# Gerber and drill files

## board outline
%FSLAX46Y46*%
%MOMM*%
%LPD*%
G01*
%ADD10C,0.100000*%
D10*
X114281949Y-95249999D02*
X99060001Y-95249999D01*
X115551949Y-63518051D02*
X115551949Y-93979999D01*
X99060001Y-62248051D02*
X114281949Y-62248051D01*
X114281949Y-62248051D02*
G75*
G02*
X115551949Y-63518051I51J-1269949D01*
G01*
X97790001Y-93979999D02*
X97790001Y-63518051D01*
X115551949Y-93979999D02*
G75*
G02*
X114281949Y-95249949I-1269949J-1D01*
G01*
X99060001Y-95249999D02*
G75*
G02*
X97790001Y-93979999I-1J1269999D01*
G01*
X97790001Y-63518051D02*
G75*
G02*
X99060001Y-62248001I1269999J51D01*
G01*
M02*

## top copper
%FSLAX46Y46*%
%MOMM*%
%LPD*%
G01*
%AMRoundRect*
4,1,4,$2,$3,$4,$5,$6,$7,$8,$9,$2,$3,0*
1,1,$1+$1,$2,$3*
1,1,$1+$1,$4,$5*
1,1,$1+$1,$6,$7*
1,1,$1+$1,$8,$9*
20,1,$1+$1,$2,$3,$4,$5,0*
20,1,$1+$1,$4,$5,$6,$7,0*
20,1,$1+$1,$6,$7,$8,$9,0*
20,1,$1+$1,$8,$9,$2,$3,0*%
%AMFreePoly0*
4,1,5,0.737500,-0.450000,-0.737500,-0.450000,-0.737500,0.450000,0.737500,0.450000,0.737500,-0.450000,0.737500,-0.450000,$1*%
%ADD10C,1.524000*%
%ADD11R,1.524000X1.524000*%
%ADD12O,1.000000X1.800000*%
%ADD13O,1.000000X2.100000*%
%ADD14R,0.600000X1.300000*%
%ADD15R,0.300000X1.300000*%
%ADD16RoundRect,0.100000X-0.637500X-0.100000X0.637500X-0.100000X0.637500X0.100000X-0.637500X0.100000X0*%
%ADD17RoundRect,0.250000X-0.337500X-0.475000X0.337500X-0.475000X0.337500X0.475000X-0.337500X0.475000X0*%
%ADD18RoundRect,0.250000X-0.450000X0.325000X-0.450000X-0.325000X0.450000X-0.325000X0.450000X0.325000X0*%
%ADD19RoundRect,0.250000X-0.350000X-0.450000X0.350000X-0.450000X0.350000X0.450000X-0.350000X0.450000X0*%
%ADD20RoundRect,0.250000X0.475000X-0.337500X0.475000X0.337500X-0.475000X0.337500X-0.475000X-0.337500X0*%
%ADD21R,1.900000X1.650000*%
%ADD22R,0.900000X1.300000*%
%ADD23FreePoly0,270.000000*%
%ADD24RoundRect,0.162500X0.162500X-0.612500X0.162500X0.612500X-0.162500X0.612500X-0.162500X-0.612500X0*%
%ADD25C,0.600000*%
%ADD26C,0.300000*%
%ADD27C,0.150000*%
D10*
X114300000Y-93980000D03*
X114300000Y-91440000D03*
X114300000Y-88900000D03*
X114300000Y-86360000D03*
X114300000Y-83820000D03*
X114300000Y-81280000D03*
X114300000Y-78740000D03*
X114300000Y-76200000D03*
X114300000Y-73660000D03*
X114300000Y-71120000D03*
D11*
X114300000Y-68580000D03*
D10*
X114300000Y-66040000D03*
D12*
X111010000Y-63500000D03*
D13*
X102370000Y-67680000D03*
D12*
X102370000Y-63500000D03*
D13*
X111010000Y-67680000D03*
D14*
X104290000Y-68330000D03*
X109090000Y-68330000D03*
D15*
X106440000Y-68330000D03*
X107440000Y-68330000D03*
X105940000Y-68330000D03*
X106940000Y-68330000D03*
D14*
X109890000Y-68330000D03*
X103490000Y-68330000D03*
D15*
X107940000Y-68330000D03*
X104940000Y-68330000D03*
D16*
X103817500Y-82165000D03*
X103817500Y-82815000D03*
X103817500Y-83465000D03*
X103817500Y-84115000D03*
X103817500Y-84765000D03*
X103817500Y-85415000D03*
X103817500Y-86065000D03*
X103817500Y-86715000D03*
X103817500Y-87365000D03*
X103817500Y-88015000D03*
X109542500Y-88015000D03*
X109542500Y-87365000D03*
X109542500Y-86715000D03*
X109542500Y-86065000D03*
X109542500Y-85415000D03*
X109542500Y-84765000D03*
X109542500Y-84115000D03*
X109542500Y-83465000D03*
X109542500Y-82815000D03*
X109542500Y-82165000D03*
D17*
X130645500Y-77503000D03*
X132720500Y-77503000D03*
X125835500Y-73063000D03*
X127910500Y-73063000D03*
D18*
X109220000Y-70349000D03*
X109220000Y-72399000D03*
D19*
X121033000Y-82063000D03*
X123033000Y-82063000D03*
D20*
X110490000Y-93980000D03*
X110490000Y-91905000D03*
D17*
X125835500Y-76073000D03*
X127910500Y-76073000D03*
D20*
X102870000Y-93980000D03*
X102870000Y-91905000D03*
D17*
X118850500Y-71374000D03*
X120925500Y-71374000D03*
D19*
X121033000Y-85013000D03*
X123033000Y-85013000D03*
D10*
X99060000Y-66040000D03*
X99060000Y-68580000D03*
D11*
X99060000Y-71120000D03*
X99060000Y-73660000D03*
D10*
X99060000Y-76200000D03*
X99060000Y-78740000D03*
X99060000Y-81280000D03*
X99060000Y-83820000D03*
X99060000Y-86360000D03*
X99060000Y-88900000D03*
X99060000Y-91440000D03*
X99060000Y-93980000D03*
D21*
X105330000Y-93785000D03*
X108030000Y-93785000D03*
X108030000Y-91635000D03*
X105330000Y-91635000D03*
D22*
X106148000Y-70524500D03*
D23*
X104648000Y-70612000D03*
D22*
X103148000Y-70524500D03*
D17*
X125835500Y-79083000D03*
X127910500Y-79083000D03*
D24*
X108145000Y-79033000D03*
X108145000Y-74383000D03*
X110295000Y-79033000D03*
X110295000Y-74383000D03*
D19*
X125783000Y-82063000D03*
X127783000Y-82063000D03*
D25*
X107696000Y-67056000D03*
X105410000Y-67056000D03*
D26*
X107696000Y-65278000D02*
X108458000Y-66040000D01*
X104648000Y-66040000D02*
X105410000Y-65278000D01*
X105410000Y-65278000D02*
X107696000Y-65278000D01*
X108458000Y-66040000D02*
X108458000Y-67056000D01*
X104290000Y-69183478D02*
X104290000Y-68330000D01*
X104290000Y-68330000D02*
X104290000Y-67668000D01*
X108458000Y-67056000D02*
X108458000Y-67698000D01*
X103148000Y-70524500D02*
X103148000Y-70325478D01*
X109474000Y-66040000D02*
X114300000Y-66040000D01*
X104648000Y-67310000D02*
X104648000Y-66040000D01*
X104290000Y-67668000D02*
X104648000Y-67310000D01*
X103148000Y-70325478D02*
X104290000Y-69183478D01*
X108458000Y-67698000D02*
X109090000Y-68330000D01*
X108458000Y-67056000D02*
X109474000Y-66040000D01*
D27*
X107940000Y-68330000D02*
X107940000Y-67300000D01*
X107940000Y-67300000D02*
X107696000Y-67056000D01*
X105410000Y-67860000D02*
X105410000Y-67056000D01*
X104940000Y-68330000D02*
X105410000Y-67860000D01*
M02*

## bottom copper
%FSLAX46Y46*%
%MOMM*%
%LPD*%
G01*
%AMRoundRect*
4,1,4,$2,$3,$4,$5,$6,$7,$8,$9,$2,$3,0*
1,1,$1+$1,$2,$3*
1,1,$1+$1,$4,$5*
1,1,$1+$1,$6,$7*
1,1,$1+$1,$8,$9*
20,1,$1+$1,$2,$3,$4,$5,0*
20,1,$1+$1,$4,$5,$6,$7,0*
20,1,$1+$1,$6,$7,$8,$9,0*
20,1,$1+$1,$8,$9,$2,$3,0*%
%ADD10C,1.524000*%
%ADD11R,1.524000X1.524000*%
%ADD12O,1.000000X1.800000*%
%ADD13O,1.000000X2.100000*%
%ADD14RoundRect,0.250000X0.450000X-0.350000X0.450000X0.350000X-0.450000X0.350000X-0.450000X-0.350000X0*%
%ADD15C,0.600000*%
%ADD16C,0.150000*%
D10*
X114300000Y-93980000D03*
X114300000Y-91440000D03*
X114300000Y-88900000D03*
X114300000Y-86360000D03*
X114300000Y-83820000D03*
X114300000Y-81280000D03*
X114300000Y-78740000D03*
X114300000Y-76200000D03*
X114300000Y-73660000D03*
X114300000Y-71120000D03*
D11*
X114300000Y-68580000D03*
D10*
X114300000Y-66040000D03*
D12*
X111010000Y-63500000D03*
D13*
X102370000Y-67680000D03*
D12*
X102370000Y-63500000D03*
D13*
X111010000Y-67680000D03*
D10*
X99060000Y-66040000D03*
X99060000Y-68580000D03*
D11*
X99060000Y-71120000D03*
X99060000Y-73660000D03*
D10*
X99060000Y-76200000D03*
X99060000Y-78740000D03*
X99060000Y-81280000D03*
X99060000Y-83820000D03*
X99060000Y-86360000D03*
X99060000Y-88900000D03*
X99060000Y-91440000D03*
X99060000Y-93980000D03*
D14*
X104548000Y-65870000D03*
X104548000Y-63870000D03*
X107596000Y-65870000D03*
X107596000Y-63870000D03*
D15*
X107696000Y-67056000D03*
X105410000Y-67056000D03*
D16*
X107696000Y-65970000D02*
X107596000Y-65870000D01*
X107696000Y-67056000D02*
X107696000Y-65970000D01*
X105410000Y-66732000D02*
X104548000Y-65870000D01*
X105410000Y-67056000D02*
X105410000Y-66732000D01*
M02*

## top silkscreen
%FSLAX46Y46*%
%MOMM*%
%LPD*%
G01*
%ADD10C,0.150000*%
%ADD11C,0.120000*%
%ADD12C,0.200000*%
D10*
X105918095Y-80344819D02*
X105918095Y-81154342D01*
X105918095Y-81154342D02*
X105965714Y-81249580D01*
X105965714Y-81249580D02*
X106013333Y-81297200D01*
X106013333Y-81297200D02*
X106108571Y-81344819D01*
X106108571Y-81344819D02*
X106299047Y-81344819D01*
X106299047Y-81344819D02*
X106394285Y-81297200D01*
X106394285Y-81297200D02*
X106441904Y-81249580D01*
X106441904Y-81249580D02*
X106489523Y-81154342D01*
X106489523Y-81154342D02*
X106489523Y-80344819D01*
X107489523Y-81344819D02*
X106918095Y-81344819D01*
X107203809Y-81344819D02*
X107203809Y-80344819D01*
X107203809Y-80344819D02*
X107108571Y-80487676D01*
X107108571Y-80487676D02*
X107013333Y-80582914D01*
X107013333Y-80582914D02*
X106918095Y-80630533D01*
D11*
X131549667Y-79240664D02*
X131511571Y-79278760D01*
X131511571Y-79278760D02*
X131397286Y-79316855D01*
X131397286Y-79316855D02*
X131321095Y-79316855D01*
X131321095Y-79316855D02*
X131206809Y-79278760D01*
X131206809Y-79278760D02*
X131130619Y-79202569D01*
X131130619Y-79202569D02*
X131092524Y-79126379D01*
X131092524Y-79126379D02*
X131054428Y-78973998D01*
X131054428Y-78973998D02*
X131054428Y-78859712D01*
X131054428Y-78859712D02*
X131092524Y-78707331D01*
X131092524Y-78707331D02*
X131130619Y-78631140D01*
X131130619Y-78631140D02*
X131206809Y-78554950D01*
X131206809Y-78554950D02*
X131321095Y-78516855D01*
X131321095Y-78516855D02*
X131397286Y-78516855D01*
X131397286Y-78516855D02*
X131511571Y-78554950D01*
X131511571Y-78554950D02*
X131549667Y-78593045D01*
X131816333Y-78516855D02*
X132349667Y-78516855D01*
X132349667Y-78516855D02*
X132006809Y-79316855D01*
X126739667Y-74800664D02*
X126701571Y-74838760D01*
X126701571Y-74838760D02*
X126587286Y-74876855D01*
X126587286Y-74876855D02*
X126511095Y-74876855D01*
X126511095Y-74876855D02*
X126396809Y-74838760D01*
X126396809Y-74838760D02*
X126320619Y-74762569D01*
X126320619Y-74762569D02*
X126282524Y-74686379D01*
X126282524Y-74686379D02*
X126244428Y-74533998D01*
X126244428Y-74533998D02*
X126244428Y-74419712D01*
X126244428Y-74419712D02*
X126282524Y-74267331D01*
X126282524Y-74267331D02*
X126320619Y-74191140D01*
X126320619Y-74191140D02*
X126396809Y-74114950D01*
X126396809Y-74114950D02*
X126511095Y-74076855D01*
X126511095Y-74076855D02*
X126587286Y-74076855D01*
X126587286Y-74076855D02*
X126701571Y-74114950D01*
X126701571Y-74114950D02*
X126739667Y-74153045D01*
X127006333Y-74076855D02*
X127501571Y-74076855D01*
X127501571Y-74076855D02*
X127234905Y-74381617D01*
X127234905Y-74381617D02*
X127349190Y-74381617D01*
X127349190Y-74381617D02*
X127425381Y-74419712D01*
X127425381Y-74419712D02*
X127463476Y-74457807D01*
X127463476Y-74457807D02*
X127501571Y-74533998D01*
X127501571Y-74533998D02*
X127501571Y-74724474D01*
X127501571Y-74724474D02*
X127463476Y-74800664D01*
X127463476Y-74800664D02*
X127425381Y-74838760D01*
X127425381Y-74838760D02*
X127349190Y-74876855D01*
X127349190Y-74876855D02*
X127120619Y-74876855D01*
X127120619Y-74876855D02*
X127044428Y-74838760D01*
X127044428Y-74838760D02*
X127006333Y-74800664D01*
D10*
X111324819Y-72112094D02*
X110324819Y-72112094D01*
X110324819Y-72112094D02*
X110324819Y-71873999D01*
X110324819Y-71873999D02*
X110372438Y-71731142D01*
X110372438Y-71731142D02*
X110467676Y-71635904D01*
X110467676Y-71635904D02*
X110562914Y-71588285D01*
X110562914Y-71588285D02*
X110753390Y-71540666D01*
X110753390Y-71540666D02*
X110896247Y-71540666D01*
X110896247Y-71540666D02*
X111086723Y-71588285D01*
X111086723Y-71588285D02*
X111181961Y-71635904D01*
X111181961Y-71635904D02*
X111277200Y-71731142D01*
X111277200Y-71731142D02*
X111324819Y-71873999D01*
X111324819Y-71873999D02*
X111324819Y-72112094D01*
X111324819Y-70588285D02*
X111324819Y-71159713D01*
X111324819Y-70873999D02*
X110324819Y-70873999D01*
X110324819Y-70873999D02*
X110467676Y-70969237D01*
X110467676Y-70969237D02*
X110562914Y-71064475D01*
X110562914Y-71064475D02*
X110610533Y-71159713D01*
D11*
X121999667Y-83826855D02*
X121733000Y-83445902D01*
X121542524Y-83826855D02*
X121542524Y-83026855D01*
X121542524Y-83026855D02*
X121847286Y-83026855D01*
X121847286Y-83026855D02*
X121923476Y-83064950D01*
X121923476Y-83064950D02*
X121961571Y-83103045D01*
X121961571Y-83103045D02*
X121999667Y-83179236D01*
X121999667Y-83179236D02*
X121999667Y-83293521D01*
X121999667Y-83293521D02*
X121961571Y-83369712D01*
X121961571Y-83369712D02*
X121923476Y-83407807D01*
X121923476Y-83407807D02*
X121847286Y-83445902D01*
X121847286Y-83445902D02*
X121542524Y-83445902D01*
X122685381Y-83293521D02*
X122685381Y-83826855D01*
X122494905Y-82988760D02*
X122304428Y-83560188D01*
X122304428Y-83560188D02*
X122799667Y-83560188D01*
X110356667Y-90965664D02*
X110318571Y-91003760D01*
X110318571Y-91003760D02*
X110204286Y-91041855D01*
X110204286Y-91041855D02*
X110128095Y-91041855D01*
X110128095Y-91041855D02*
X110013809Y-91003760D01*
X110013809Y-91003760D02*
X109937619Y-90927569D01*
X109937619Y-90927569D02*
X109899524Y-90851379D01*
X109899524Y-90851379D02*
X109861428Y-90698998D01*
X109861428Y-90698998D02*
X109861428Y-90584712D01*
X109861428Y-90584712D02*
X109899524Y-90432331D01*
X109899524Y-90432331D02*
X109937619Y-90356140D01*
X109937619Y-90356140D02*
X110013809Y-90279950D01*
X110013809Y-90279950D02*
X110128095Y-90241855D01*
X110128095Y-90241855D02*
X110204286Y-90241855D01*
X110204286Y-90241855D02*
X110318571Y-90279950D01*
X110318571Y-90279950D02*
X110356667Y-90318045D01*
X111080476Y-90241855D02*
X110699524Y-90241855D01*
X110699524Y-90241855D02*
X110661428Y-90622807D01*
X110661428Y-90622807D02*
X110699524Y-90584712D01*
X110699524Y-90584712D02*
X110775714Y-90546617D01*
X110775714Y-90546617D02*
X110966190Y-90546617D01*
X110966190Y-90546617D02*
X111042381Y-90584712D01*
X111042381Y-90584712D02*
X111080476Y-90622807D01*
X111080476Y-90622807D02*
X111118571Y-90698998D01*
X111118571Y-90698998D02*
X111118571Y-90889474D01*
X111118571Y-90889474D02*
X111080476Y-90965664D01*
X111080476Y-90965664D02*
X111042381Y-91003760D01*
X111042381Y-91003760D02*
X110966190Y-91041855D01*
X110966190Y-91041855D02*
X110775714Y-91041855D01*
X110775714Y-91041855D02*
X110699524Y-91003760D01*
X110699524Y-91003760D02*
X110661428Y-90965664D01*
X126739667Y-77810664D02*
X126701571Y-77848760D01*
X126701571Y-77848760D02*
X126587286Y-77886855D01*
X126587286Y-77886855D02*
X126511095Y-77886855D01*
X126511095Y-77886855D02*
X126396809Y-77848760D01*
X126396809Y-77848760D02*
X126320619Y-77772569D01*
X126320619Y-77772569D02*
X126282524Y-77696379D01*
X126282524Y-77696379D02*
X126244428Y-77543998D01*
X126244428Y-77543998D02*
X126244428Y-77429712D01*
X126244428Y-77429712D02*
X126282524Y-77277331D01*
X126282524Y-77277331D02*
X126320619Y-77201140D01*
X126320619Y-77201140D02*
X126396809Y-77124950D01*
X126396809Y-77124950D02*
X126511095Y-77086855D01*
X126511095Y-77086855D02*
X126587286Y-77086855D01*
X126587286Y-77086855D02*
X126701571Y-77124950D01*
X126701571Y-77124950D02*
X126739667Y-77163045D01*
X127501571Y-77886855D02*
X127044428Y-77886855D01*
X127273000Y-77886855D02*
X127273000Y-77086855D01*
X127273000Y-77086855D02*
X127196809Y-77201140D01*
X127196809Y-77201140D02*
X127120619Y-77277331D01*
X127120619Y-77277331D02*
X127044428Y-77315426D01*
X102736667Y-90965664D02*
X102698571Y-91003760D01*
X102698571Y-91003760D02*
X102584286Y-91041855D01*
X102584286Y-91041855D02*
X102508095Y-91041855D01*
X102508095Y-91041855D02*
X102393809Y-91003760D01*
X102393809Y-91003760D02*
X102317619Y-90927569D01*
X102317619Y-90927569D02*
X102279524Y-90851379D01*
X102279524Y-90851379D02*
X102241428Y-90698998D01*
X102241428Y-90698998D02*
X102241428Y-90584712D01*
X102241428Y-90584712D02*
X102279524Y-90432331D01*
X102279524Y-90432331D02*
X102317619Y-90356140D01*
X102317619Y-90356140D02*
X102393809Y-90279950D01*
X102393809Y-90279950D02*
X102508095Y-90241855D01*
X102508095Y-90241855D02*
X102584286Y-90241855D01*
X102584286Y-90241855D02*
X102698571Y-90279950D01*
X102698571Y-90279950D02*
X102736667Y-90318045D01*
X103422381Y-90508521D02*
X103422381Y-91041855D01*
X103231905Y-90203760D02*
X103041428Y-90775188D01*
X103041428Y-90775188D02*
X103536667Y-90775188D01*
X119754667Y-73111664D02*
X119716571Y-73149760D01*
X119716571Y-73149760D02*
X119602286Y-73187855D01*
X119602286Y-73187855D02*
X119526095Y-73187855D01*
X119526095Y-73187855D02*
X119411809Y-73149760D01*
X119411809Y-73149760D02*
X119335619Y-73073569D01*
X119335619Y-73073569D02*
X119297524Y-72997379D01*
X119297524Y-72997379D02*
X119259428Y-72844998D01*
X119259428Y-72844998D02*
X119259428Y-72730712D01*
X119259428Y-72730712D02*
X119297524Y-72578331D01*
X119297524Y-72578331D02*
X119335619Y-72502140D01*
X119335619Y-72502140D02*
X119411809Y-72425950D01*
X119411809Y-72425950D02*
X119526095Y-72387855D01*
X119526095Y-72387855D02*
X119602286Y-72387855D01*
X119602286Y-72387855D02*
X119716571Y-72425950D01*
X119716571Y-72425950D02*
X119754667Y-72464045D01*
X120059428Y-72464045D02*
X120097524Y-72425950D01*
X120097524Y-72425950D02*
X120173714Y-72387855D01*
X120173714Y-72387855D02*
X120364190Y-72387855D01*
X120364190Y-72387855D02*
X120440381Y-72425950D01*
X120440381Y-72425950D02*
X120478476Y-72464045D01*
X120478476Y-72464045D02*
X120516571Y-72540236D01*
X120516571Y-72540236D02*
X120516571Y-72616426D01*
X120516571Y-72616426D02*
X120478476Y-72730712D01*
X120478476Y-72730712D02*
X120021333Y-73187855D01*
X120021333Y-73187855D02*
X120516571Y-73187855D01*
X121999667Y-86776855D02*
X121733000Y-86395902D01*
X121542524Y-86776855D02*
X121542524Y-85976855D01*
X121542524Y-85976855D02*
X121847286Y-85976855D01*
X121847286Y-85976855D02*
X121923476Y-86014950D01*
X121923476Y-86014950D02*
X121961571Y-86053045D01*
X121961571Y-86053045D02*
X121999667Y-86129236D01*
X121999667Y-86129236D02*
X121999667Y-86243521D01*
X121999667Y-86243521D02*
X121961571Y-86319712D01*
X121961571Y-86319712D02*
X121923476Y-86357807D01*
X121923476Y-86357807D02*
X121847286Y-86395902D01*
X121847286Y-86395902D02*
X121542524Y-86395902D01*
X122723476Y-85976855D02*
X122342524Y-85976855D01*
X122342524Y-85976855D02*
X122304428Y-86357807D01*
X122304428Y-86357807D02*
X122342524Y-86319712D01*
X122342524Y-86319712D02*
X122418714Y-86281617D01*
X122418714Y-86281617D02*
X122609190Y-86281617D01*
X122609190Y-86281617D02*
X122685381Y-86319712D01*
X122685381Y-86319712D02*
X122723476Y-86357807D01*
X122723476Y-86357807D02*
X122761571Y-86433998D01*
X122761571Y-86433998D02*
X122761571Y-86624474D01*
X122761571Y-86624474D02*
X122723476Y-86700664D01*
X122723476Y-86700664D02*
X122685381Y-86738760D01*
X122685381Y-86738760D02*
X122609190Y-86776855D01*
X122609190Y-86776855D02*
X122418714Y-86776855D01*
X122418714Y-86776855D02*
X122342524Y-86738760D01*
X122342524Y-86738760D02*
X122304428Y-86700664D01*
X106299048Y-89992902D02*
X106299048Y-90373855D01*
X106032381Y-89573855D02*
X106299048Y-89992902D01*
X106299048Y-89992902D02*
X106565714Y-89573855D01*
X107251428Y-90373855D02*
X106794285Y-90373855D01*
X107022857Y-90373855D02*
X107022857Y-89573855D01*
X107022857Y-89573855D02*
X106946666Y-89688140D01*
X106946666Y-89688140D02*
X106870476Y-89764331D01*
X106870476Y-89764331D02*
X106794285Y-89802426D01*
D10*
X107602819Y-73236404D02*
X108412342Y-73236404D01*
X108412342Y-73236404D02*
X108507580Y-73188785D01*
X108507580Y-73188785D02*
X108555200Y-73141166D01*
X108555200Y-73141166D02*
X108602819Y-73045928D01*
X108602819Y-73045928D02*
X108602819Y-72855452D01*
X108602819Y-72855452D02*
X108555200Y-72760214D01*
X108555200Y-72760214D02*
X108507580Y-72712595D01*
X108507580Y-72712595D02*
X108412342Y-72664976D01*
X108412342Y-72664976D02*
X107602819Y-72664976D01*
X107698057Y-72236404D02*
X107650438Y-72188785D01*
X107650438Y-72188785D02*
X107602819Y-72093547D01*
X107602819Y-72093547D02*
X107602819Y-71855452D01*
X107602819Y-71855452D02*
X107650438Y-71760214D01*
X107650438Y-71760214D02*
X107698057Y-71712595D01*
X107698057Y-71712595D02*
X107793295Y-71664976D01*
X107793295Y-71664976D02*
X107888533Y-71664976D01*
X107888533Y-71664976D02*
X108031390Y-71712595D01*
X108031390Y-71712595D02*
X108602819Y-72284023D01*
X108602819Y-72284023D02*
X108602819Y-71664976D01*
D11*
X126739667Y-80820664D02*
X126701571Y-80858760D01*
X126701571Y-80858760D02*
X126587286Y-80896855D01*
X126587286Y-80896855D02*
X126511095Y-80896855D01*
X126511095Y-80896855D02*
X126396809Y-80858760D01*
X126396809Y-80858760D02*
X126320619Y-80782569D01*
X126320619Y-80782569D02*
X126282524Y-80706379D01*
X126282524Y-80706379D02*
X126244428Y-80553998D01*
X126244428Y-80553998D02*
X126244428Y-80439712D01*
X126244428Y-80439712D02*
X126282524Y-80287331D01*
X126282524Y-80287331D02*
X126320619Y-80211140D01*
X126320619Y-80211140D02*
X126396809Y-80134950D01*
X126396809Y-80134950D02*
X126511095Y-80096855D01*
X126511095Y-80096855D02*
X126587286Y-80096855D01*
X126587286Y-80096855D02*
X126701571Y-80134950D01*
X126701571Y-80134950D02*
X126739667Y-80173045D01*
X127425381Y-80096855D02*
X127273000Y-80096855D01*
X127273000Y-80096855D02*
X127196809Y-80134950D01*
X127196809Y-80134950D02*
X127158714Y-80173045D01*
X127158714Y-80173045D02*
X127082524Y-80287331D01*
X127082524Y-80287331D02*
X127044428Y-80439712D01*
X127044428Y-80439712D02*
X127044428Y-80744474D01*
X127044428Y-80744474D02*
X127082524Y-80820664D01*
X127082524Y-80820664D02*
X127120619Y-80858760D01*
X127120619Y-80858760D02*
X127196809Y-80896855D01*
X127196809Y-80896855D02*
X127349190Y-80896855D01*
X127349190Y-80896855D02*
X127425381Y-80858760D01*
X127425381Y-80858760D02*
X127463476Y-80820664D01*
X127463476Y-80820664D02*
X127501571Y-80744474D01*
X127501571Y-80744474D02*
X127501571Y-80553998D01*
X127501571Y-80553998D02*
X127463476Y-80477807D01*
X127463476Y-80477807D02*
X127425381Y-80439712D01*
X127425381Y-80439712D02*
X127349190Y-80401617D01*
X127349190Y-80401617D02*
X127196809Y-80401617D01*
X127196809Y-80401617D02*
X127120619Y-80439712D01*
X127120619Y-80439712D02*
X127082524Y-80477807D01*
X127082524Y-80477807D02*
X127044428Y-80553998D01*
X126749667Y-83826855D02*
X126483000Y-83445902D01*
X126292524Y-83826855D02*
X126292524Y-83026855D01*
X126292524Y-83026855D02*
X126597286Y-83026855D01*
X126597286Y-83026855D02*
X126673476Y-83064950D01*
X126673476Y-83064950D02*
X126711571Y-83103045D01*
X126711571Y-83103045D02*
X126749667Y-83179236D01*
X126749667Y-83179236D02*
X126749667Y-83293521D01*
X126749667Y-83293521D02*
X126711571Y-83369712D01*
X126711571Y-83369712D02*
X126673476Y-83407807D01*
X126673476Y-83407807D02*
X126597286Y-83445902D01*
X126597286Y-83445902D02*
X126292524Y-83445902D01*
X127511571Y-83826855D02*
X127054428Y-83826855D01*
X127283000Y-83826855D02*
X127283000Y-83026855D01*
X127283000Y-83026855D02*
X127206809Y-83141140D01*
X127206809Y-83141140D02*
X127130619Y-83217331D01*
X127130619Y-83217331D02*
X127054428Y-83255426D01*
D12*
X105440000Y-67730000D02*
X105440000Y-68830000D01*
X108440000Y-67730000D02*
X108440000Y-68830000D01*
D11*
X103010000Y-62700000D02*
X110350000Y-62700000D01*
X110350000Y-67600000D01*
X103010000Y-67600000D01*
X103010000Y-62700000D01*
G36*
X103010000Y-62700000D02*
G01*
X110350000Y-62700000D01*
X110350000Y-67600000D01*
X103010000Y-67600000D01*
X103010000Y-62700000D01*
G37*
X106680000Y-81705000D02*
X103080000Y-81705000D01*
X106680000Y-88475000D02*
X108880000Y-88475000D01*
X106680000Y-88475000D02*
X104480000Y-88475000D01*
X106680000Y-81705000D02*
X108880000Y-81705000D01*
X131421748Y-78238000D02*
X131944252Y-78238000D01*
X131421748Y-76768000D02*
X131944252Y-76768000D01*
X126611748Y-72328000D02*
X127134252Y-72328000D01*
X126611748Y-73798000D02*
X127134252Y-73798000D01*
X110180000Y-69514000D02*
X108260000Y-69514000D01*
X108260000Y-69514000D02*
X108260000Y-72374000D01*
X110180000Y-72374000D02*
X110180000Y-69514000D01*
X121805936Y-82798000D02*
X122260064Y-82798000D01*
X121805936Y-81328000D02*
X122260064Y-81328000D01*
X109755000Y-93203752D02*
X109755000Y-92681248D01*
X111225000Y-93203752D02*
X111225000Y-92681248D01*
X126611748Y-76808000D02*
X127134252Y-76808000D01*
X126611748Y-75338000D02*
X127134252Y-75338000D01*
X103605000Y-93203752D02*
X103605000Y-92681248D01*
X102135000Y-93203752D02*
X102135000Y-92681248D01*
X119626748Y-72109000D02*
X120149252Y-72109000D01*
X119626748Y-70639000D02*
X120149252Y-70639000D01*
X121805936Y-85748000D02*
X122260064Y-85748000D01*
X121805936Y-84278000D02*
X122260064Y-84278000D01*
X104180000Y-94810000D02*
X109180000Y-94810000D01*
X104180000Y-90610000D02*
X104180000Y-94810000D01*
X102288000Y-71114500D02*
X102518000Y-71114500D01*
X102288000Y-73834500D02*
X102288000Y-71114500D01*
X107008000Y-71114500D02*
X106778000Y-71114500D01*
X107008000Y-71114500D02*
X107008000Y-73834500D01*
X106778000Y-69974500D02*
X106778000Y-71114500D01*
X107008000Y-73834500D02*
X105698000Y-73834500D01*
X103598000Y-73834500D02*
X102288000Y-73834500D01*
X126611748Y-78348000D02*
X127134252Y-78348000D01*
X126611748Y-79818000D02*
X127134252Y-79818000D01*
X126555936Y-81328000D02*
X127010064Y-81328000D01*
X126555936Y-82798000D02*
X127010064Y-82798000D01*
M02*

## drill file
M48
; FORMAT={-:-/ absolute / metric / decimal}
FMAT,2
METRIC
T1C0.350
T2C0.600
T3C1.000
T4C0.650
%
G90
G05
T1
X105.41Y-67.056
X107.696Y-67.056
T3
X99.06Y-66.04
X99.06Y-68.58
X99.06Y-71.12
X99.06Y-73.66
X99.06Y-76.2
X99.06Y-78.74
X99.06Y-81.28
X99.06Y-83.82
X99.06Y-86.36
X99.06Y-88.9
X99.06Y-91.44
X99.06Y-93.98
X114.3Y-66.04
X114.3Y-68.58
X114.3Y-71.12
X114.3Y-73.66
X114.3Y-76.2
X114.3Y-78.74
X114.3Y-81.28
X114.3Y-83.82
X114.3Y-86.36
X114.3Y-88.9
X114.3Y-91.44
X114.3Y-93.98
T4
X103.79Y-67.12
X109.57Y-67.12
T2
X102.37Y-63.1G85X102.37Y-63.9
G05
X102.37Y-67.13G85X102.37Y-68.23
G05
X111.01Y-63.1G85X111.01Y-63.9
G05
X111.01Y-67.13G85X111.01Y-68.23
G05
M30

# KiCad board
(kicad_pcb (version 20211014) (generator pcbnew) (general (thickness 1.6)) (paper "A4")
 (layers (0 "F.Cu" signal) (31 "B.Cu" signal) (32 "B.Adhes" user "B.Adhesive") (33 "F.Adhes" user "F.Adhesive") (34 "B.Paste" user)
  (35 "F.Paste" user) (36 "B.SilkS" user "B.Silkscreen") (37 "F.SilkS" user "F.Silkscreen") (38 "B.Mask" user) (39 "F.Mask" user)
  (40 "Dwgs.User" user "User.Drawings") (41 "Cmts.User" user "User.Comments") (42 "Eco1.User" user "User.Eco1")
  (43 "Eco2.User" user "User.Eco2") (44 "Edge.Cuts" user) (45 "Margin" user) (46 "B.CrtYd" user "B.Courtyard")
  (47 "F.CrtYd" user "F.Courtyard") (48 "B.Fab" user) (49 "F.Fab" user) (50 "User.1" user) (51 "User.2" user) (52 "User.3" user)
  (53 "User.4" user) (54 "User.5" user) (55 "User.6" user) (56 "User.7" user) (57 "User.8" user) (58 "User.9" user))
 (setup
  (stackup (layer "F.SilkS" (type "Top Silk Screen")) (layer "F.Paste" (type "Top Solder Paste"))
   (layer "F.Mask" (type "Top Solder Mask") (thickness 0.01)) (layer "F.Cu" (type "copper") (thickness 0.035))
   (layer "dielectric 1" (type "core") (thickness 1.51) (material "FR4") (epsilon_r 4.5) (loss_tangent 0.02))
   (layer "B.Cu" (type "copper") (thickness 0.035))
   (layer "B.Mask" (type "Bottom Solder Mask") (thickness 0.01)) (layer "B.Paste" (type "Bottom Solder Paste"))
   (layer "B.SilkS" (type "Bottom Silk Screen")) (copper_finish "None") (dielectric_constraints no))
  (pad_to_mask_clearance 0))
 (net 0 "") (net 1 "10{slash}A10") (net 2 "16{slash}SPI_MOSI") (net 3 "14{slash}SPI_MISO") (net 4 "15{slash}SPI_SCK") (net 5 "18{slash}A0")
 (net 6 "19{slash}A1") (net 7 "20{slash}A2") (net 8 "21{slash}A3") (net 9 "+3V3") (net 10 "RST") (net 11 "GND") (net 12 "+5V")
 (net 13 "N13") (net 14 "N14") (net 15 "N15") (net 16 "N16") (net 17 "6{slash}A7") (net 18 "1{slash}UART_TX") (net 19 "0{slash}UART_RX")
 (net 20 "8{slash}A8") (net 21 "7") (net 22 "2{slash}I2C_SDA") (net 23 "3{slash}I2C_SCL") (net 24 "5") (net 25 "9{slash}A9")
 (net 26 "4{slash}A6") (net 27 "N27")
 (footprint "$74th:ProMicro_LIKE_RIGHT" (layer "F.Cu") (at 114.3 81.28)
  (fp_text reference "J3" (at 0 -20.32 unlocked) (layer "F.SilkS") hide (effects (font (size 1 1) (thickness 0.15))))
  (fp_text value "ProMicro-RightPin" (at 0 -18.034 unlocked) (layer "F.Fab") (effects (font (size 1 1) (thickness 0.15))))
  (pad "1" thru_hole circle (at 0 12.7 180) (size 1.524 1.524) (drill 1) (layers *.Cu *.Mask) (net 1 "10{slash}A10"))
  (pad "2" thru_hole circle (at 0 10.16) (size 1.524 1.524) (drill 1) (layers *.Cu *.Mask) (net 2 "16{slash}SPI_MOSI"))
  (pad "3" thru_hole circle (at 0 7.62 180) (size 1.524 1.524) (drill 1) (layers *.Cu *.Mask) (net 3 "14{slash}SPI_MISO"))
  (pad "4" thru_hole circle (at 0 5.08 180) (size 1.524 1.524) (drill 1) (layers *.Cu *.Mask) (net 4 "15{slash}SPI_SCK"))
  (pad "5" thru_hole circle (at 0 2.54 180) (size 1.524 1.524) (drill 1) (layers *.Cu *.Mask) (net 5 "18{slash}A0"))
  (pad "6" thru_hole circle (at 0 0 180) (size 1.524 1.524) (drill 1) (layers *.Cu *.Mask) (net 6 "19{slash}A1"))
  (pad "7" thru_hole circle (at 0 -2.54 180) (size 1.524 1.524) (drill 1) (layers *.Cu *.Mask) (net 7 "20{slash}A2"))
  (pad "8" thru_hole circle (at 0 -5.08 180) (size 1.524 1.524) (drill 1) (layers *.Cu *.Mask) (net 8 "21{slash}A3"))
  (pad "9" thru_hole circle (at 0 -7.62 180) (size 1.524 1.524) (drill 1) (layers *.Cu *.Mask) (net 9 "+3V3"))
  (pad "10" thru_hole circle (at 0 -10.16 180) (size 1.524 1.524) (drill 1) (layers *.Cu *.Mask) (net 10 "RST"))
  (pad "11" thru_hole rect (at 0 -12.7 180) (size 1.524 1.524) (drill 1) (layers *.Cu *.Mask) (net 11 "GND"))
  (pad "12" thru_hole circle (at 0 -15.24 180) (size 1.524 1.524) (drill 1) (layers *.Cu *.Mask) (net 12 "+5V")))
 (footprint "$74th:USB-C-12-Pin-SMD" (layer "F.Cu") (at 106.68 63.5 180)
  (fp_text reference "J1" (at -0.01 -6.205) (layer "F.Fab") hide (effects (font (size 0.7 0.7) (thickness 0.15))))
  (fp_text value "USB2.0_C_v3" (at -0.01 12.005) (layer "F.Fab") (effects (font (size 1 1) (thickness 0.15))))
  (fp_line (start 1.24 -4.23) (end 1.24 -5.33) (layer "F.SilkS") (width 0.2))
  (fp_line (start -1.76 -4.23) (end -1.76 -5.33) (layer "F.SilkS") (width 0.2))
  (fp_rect (start -3.67 -4.1) (end 3.67 0.8) (layer "F.SilkS") (width 0.12) (fill solid))
  (pad "" thru_hole oval (at -4.33 0) (size 1 1.8) (drill oval 0.6 1.4) (layers *.Cu *.Mask))
  (pad "" np_thru_hole circle (at 2.89 -3.62) (size 0.65 0.65) (drill 0.65) (layers *.Mask))
  (pad "" thru_hole oval (at 4.31 -4.18) (size 1 2.1) (drill oval 0.6 1.7) (layers *.Cu *.Mask))
  (pad "" np_thru_hole circle (at -2.89 -3.62) (size 0.65 0.65) (drill 0.65) (layers *.Mask))
  (pad "" thru_hole oval (at 4.31 0) (size 1 1.8) (drill oval 0.6 1.4) (layers *.Cu *.Mask))
  (pad "" thru_hole oval (at -4.33 -4.18) (size 1 2.1) (drill oval 0.6 1.7) (layers *.Cu *.Mask))
  (pad "1" smd rect (at 2.39 -4.83) (size 0.6 1.3) (layers "F.Cu" "F.Paste" "F.Mask") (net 12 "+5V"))
  (pad "1" smd rect (at -2.41 -4.83) (size 0.6 1.3) (layers "F.Cu" "F.Paste" "F.Mask") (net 12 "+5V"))
  (pad "2" smd rect (at 0.24 -4.83) (size 0.3 1.3) (layers "F.Cu" "F.Paste" "F.Mask") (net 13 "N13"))
  (pad "2" smd rect (at -0.76 -4.83) (size 0.3 1.3) (layers "F.Cu" "F.Paste" "F.Mask") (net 13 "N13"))
  (pad "3" smd rect (at 0.74 -4.83) (size 0.3 1.3) (layers "F.Cu" "F.Paste" "F.Mask") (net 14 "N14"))
  (pad "3" smd rect (at -0.26 -4.83) (size 0.3 1.3) (layers "F.Cu" "F.Paste" "F.Mask") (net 14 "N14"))
  (pad "4" smd rect (at -3.21 -4.83) (size 0.6 1.3) (layers "F.Cu" "F.Paste" "F.Mask") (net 11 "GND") (zone_connect 2))
  (pad "4" smd rect (at 3.19 -4.83) (size 0.6 1.3) (layers "F.Cu" "F.Paste" "F.Mask") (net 11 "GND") (zone_connect 2))
  (pad "5" smd rect (at -1.26 -4.83) (size 0.3 1.3) (layers "F.Cu" "F.Paste" "F.Mask") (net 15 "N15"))
  (pad "6" smd rect (at 1.74 -4.83) (size 0.3 1.3) (layers "F.Cu" "F.Paste" "F.Mask") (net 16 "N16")))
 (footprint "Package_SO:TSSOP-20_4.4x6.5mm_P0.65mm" (layer "F.Cu") (at 106.68 85.09)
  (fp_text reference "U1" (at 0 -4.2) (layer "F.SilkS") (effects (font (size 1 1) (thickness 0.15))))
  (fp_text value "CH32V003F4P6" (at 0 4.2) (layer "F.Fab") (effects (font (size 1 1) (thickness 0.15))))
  (fp_line (start 0 -3.385) (end -3.6 -3.385) (layer "F.SilkS") (width 0.12))
  (fp_line (start 0 3.385) (end 2.2 3.385) (layer "F.SilkS") (width 0.12))
  (fp_line (start 0 3.385) (end -2.2 3.385) (layer "F.SilkS") (width 0.12))
  (fp_line (start 0 -3.385) (end 2.2 -3.385) (layer "F.SilkS") (width 0.12))
  (pad "1" smd roundrect locked (at -2.8625 -2.925) (size 1.475 0.4) (layers "F.Cu" "F.Paste" "F.Mask") (roundrect_rratio 0.25)
   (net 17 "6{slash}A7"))
  (pad "2" smd roundrect locked (at -2.8625 -2.275) (size 1.475 0.4) (layers "F.Cu" "F.Paste" "F.Mask") (roundrect_rratio 0.25)
   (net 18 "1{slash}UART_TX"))
  (pad "3" smd roundrect locked (at -2.8625 -1.625) (size 1.475 0.4) (layers "F.Cu" "F.Paste" "F.Mask") (roundrect_rratio 0.25)
   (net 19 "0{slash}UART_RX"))
  (pad "4" smd roundrect locked (at -2.8625 -0.975) (size 1.475 0.4) (layers "F.Cu" "F.Paste" "F.Mask") (roundrect_rratio 0.25)
   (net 10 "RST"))
  (pad "5" smd roundrect locked (at -2.8625 -0.325) (size 1.475 0.4) (layers "F.Cu" "F.Paste" "F.Mask") (roundrect_rratio 0.25)
   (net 6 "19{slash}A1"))
  (pad "6" smd roundrect locked (at -2.8625 0.325) (size 1.475 0.4) (layers "F.Cu" "F.Paste" "F.Mask") (roundrect_rratio 0.25)
   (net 5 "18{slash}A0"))
  (pad "7" smd roundrect locked (at -2.8625 0.975) (size 1.475 0.4) (layers "F.Cu" "F.Paste" "F.Mask") (roundrect_rratio 0.25)
   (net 11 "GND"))
  (pad "8" smd roundrect locked (at -2.8625 1.625) (size 1.475 0.4) (layers "F.Cu" "F.Paste" "F.Mask") (roundrect_rratio 0.25)
   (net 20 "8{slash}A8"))
  (pad "9" smd roundrect locked (at -2.8625 2.275) (size 1.475 0.4) (layers "F.Cu" "F.Paste" "F.Mask") (roundrect_rratio 0.25)
   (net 9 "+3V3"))
  (pad "10" smd roundrect locked (at -2.8625 2.925) (size 1.475 0.4) (layers "F.Cu" "F.Paste" "F.Mask") (roundrect_rratio 0.25) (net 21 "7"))
  (pad "11" smd roundrect locked (at 2.8625 2.925) (size 1.475 0.4) (layers "F.Cu" "F.Paste" "F.Mask") (roundrect_rratio 0.25)
   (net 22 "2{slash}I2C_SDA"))
  (pad "12" smd roundrect locked (at 2.8625 2.275) (size 1.475 0.4) (layers "F.Cu" "F.Paste" "F.Mask") (roundrect_rratio 0.25)
   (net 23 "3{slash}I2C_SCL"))
  (pad "13" smd roundrect locked (at 2.8625 1.625) (size 1.475 0.4) (layers "F.Cu" "F.Paste" "F.Mask") (roundrect_rratio 0.25) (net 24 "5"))
  (pad "14" smd roundrect locked (at 2.8625 0.975) (size 1.475 0.4) (layers "F.Cu" "F.Paste" "F.Mask") (roundrect_rratio 0.25)
   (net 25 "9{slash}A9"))
  (pad "15" smd roundrect locked (at 2.8625 0.325) (size 1.475 0.4) (layers "F.Cu" "F.Paste" "F.Mask") (roundrect_rratio 0.25)
   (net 4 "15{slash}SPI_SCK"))
  (pad "16" smd roundrect locked (at 2.8625 -0.325) (size 1.475 0.4) (layers "F.Cu" "F.Paste" "F.Mask") (roundrect_rratio 0.25)
   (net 2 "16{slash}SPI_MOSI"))
  (pad "17" smd roundrect locked (at 2.8625 -0.975) (size 1.475 0.4) (layers "F.Cu" "F.Paste" "F.Mask") (roundrect_rratio 0.25)
   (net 3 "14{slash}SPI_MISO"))
  (pad "18" smd roundrect locked (at 2.8625 -1.625) (size 1.475 0.4) (layers "F.Cu" "F.Paste" "F.Mask") (roundrect_rratio 0.25)
   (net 8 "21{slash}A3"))
  (pad "19" smd roundrect locked (at 2.8625 -2.275) (size 1.475 0.4) (layers "F.Cu" "F.Paste" "F.Mask") (roundrect_rratio 0.25)
   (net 1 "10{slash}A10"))
  (pad "20" smd roundrect locked (at 2.8625 -2.925) (size 1.475 0.4) (layers "F.Cu" "F.Paste" "F.Mask") (roundrect_rratio 0.25)
   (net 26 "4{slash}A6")))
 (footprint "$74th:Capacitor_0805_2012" (layer "F.Cu") (at 131.683 77.503)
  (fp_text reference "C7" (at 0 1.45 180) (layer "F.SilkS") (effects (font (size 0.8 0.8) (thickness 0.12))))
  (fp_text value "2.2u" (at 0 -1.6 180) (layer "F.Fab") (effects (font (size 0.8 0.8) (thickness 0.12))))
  (fp_line (start -0.261252 0.735) (end 0.261252 0.735) (layer "F.SilkS") (width 0.12))
  (fp_line (start -0.261252 -0.735) (end 0.261252 -0.735) (layer "F.SilkS") (width 0.12))
  (pad "1" smd roundrect (at -1.0375 0) (size 1.175 1.45) (layers "F.Cu" "F.Paste" "F.Mask") (roundrect_rratio 0.212766) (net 9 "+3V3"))
  (pad "2" smd roundrect (at 1.0375 0) (size 1.175 1.45) (layers "F.Cu" "F.Paste" "F.Mask") (roundrect_rratio 0.212766) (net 11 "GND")))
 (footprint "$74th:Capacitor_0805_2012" (layer "F.Cu") (at 126.873 73.063)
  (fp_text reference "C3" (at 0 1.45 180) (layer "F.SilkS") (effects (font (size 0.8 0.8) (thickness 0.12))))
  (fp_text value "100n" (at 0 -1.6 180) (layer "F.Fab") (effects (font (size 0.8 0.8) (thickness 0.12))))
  (fp_line (start -0.261252 -0.735) (end 0.261252 -0.735) (layer "F.SilkS") (width 0.12))
  (fp_line (start -0.261252 0.735) (end 0.261252 0.735) (layer "F.SilkS") (width 0.12))
  (pad "1" smd roundrect (at -1.0375 0) (size 1.175 1.45) (layers "F.Cu" "F.Paste" "F.Mask") (roundrect_rratio 0.212766) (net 9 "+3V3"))
  (pad "2" smd roundrect (at 1.0375 0) (size 1.175 1.45) (layers "F.Cu" "F.Paste" "F.Mask") (roundrect_rratio 0.212766) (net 11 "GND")))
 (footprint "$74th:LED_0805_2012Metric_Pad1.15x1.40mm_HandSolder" (layer "F.Cu") (at 109.22 71.374 -90)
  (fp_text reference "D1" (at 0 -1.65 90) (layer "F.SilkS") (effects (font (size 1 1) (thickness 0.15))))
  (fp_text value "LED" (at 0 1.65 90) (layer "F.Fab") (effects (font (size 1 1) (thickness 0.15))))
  (fp_line (start -1.86 -0.96) (end -1.86 0.96) (layer "F.SilkS") (width 0.12))
  (fp_line (start -1.86 0.96) (end 1 0.96) (layer "F.SilkS") (width 0.12))
  (fp_line (start 1 -0.96) (end -1.86 -0.96) (layer "F.SilkS") (width 0.12))
  (pad "1" smd roundrect (at -1.025 0 270) (size 1.15 1.4) (layers "F.Cu" "F.Paste" "F.Mask") (roundrect_rratio 0.217391) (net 11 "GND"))
  (pad "2" smd roundrect (at 1.025 0 270) (size 1.15 1.4) (layers "F.Cu" "F.Paste" "F.Mask") (roundrect_rratio 0.217391) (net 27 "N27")))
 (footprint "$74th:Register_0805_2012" (layer "F.Cu") (at 122.133 81.963)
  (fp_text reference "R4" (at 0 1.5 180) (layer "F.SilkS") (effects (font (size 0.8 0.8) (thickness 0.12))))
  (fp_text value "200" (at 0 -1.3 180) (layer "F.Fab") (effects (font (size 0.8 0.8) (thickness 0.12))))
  (fp_line (start -0.327064 0.835) (end 0.127064 0.835) (layer "F.SilkS") (width 0.12))
  (fp_line (start -0.327064 -0.635) (end 0.127064 -0.635) (layer "F.SilkS") (width 0.12))
  (pad "1" smd roundrect (at -1.1 0.1) (size 1.2 1.4) (layers "F.Cu" "F.Paste" "F.Mask") (roundrect_rratio 0.208333) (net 9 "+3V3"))
  (pad "2" smd roundrect (at 0.9 0.1) (size 1.2 1.4) (layers "F.Cu" "F.Paste" "F.Mask") (roundrect_rratio 0.208333) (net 27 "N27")))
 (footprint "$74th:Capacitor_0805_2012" (layer "F.Cu") (at 110.49 92.9425 90)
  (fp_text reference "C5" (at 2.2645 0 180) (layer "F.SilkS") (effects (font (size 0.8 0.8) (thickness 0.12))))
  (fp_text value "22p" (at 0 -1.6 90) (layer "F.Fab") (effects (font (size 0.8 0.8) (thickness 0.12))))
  (fp_line (start -0.261252 -0.735) (end 0.261252 -0.735) (layer "F.SilkS") (width 0.12))
  (fp_line (start -0.261252 0.735) (end 0.261252 0.735) (layer "F.SilkS") (width 0.12))
  (pad "1" smd roundrect (at -1.0375 0 90) (size 1.175 1.45) (layers "F.Cu" "F.Paste" "F.Mask") (roundrect_rratio 0.212766)
   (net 6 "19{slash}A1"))
  (pad "2" smd roundrect (at 1.0375 0 90) (size 1.175 1.45) (layers "F.Cu" "F.Paste" "F.Mask") (roundrect_rratio 0.212766) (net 11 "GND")))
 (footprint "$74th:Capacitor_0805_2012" (layer "F.Cu") (at 126.873 76.073)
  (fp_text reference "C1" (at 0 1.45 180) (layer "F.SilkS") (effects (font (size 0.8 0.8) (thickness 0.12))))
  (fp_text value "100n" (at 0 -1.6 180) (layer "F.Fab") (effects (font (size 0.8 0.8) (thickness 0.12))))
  (fp_line (start -0.261252 0.735) (end 0.261252 0.735) (layer "F.SilkS") (width 0.12))
  (fp_line (start -0.261252 -0.735) (end 0.261252 -0.735) (layer "F.SilkS") (width 0.12))
  (pad "1" smd roundrect (at -1.0375 0) (size 1.175 1.45) (layers "F.Cu" "F.Paste" "F.Mask") (roundrect_rratio 0.212766) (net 10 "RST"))
  (pad "2" smd roundrect (at 1.0375 0) (size 1.175 1.45) (layers "F.Cu" "F.Paste" "F.Mask") (roundrect_rratio 0.212766) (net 11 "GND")))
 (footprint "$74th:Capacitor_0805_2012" (layer "F.Cu") (at 102.87 92.9425 90)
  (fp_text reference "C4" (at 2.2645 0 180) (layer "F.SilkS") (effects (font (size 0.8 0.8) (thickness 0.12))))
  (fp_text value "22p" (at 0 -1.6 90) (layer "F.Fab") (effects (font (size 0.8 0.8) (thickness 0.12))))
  (fp_line (start -0.261252 0.735) (end 0.261252 0.735) (layer "F.SilkS") (width 0.12))
  (fp_line (start -0.261252 -0.735) (end 0.261252 -0.735) (layer "F.SilkS") (width 0.12))
  (pad "1" smd roundrect (at -1.0375 0 90) (size 1.175 1.45) (layers "F.Cu" "F.Paste" "F.Mask") (roundrect_rratio 0.212766)
   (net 5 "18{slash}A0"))
  (pad "2" smd roundrect (at 1.0375 0 90) (size 1.175 1.45) (layers "F.Cu" "F.Paste" "F.Mask") (roundrect_rratio 0.212766) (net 11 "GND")))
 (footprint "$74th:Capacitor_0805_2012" (layer "F.Cu") (at 119.888 71.374)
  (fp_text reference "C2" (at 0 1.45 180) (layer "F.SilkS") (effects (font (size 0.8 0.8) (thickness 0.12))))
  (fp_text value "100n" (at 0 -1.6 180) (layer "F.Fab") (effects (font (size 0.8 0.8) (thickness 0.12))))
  (fp_line (start -0.261252 0.735) (end 0.261252 0.735) (layer "F.SilkS") (width 0.12))
  (fp_line (start -0.261252 -0.735) (end 0.261252 -0.735) (layer "F.SilkS") (width 0.12))
  (pad "1" smd roundrect (at -1.0375 0) (size 1.175 1.45) (layers "F.Cu" "F.Paste" "F.Mask") (roundrect_rratio 0.212766) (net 9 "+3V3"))
  (pad "2" smd roundrect (at 1.0375 0) (size 1.175 1.45) (layers "F.Cu" "F.Paste" "F.Mask") (roundrect_rratio 0.212766) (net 11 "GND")))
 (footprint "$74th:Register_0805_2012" (layer "F.Cu") (at 122.133 84.913)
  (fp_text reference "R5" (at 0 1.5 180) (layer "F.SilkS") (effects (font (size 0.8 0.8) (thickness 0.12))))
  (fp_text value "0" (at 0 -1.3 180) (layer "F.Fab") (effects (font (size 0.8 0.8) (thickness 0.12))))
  (fp_line (start -0.327064 0.835) (end 0.127064 0.835) (layer "F.SilkS") (width 0.12))
  (fp_line (start -0.327064 -0.635) (end 0.127064 -0.635) (layer "F.SilkS") (width 0.12))
  (pad "1" smd roundrect (at -1.1 0.1) (size 1.2 1.4) (layers "F.Cu" "F.Paste" "F.Mask") (roundrect_rratio 0.208333) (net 7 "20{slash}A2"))
  (pad "2" smd roundrect (at 0.9 0.1) (size 1.2 1.4) (layers "F.Cu" "F.Paste" "F.Mask") (roundrect_rratio 0.208333) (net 11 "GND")))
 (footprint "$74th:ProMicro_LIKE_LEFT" (layer "F.Cu") (at 99.06 80.01)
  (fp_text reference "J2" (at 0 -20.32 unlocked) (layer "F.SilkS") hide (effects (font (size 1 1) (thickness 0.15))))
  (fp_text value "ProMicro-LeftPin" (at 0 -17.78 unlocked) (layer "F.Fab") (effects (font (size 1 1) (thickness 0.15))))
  (pad "1" thru_hole circle (at 0 -13.97) (size 1.524 1.524) (drill 1) (layers *.Cu *.Mask) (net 18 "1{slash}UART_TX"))
  (pad "2" thru_hole circle (at 0 -11.43 180) (size 1.524 1.524) (drill 1) (layers *.Cu *.Mask) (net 19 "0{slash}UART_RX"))
  (pad "3" thru_hole rect (at 0 -8.89) (size 1.524 1.524) (drill 1) (layers *.Cu *.Mask) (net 11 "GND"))
  (pad "4" thru_hole rect (at 0 -6.35) (size 1.524 1.524) (drill 1) (layers *.Cu *.Mask) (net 11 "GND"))
  (pad "5" thru_hole circle (at 0 -3.81) (size 1.524 1.524) (drill 1) (layers *.Cu *.Mask) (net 22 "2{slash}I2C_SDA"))
  (pad "6" thru_hole circle (at 0 -1.27) (size 1.524 1.524) (drill 1) (layers *.Cu *.Mask) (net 23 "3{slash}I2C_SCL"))
  (pad "7" thru_hole circle (at 0 1.27) (size 1.524 1.524) (drill 1) (layers *.Cu *.Mask) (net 26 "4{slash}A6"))
  (pad "8" thru_hole circle (at 0 3.81) (size 1.524 1.524) (drill 1) (layers *.Cu *.Mask) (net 24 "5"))
  (pad "9" thru_hole circle (at 0 6.35) (size 1.524 1.524) (drill 1) (layers *.Cu *.Mask) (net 17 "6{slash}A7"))
  (pad "10" thru_hole circle (at 0 8.89) (size 1.524 1.524) (drill 1) (layers *.Cu *.Mask) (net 21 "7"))
  (pad "11" thru_hole circle (at 0 11.43) (size 1.524 1.524) (drill 1) (layers *.Cu *.Mask) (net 20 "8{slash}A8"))
  (pad "12" thru_hole circle (at 0 13.97) (size 1.524 1.524) (drill 1) (layers *.Cu *.Mask) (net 25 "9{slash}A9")))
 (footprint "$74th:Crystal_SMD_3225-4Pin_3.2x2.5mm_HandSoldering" (layer "F.Cu") (at 106.68 92.71)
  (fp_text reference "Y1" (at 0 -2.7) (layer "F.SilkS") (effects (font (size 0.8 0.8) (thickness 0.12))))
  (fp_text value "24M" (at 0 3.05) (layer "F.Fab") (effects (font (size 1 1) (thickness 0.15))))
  (fp_line (start -2.5 2.1) (end 2.5 2.1) (layer "F.SilkS") (width 0.12))
  (fp_line (start -2.5 -2.1) (end -2.5 2.1) (layer "F.SilkS") (width 0.12))
  (pad "1" smd rect (at -1.35 1.075) (size 1.9 1.65) (layers "F.Cu" "F.Paste" "F.Mask") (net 6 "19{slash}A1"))
  (pad "2" smd rect (at 1.35 1.075) (size 1.9 1.65) (layers "F.Cu" "F.Paste" "F.Mask") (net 11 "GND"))
  (pad "3" smd rect (at 1.35 -1.075) (size 1.9 1.65) (layers "F.Cu" "F.Paste" "F.Mask") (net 5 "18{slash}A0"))
  (pad "4" smd rect (at -1.35 -1.075) (size 1.9 1.65) (layers "F.Cu" "F.Paste" "F.Mask") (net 11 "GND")))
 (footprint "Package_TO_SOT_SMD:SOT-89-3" (layer "F.Cu") (at 104.648 72.1745 -90)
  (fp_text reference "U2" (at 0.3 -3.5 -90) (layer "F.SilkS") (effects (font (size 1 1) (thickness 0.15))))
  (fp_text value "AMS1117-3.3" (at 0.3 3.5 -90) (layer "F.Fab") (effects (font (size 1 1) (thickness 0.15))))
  (fp_line (start -1.06 2.36) (end -1.06 2.13) (layer "F.SilkS") (width 0.12))
  (fp_line (start 1.66 2.36) (end -1.06 2.36) (layer "F.SilkS") (width 0.12))
  (fp_line (start -1.06 -2.36) (end -1.06 -2.13) (layer "F.SilkS") (width 0.12))
  (fp_line (start -1.06 -2.36) (end 1.66 -2.36) (layer "F.SilkS") (width 0.12))
  (fp_line (start -2.2 -2.13) (end -1.06 -2.13) (layer "F.SilkS") (width 0.12))
  (fp_line (start 1.66 -2.36) (end 1.66 -1.05) (layer "F.SilkS") (width 0.12))
  (fp_line (start 1.66 1.05) (end 1.66 2.36) (layer "F.SilkS") (width 0.12))
  (pad "1" smd rect locked (at -1.65 -1.5 270) (size 1.3 0.9) (layers "F.Cu" "F.Paste" "F.Mask") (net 11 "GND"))
  (pad "2" smd custom locked (at -1.5625 0 270) (size 1.475 0.9) (layers "F.Cu" "F.Paste" "F.Mask") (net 9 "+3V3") (zone_connect 2)
   (options (clearance outline) (anchor rect)) (primitives))
  (pad "3" smd rect locked (at -1.65 1.5 270) (size 1.3 0.9) (layers "F.Cu" "F.Paste" "F.Mask") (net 12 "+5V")))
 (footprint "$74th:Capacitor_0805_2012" (layer "F.Cu") (at 126.873 79.083)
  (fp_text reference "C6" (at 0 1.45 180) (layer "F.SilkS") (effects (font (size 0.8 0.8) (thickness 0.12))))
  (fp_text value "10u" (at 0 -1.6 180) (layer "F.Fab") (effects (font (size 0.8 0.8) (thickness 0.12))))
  (fp_line (start -0.261252 -0.735) (end 0.261252 -0.735) (layer "F.SilkS") (width 0.12))
  (fp_line (start -0.261252 0.735) (end 0.261252 0.735) (layer "F.SilkS") (width 0.12))
  (pad "1" smd roundrect (at -1.0375 0) (size 1.175 1.45) (layers "F.Cu" "F.Paste" "F.Mask") (roundrect_rratio 0.212766) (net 12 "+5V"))
  (pad "2" smd roundrect (at 1.0375 0) (size 1.175 1.45) (layers "F.Cu" "F.Paste" "F.Mask") (roundrect_rratio 0.212766) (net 11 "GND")))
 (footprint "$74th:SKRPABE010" (layer "F.Cu") (at 109.22 76.708 90)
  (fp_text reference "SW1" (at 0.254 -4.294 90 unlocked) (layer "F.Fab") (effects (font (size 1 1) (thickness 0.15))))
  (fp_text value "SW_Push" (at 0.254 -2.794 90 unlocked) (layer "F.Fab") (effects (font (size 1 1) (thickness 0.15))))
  (pad "1" smd roundrect (at -2.325 -1.075 90) (size 1.55 0.65) (layers "F.Cu" "F.Paste" "F.Mask") (roundrect_rratio 0.25) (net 11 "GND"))
  (pad "1" smd roundrect (at 2.325 -1.075 90) (size 1.55 0.65) (layers "F.Cu" "F.Paste" "F.Mask") (roundrect_rratio 0.25) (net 11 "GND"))
  (pad "2" smd roundrect (at -2.325 1.075 90) (size 1.55 0.65) (layers "F.Cu" "F.Paste" "F.Mask") (roundrect_rratio 0.25) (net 10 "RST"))
  (pad "2" smd roundrect (at 2.325 1.075 90) (size 1.55 0.65) (layers "F.Cu" "F.Paste" "F.Mask") (roundrect_rratio 0.25) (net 10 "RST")))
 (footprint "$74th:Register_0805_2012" (layer "F.Cu") (at 126.883 81.963)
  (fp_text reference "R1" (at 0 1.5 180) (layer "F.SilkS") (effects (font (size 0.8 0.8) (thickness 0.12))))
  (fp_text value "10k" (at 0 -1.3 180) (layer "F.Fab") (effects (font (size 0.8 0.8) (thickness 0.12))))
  (fp_line (start -0.327064 -0.635) (end 0.127064 -0.635) (layer "F.SilkS") (width 0.12))
  (fp_line (start -0.327064 0.835) (end 0.127064 0.835) (layer "F.SilkS") (width 0.12))
  (pad "1" smd roundrect (at -1.1 0.1) (size 1.2 1.4) (layers "F.Cu" "F.Paste" "F.Mask") (roundrect_rratio 0.208333) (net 9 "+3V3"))
  (pad "2" smd roundrect (at 0.9 0.1) (size 1.2 1.4) (layers "F.Cu" "F.Paste" "F.Mask") (roundrect_rratio 0.208333) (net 10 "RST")))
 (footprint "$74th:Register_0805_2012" (layer "B.Cu") (at 104.648 64.77 90)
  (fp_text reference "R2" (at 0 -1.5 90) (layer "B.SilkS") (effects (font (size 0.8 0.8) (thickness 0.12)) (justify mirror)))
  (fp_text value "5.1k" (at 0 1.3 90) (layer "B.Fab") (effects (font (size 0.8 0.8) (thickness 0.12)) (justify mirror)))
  (pad "1" smd roundrect (at -1.1 -0.1 90) (size 1.2 1.4) (layers "B.Cu" "B.Paste" "B.Mask") (roundrect_rratio 0.208333) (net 16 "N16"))
  (pad "2" smd roundrect (at 0.9 -0.1 90) (size 1.2 1.4) (layers "B.Cu" "B.Paste" "B.Mask") (roundrect_rratio 0.208333) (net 11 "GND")))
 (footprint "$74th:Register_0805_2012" (layer "B.Cu") (at 107.696 64.77 90)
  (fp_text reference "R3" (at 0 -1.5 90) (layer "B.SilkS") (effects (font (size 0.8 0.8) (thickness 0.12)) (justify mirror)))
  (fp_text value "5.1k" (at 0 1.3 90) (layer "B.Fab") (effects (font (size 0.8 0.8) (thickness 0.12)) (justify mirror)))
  (pad "1" smd roundrect (at -1.1 -0.1 90) (size 1.2 1.4) (layers "B.Cu" "B.Paste" "B.Mask") (roundrect_rratio 0.208333) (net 15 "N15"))
  (pad "2" smd roundrect (at 0.9 -0.1 90) (size 1.2 1.4) (layers "B.Cu" "B.Paste" "B.Mask") (roundrect_rratio 0.208333) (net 11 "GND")))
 (gr_line (start 114.281949 95.249999) (end 99.060001 95.249999) (layer "Edge.Cuts") (width 0.1))
 (gr_line (start 115.551949 63.518051) (end 115.551949 93.979999) (layer "Edge.Cuts") (width 0.1))
 (gr_line (start 99.060001 62.248051) (end 114.281949 62.248051) (layer "Edge.Cuts") (width 0.1))
 (gr_arc (start 114.281949 62.248051) (mid 115.179975 62.620025) (end 115.551949 63.518051) (layer "Edge.Cuts") (width 0.1))
 (gr_line (start 97.790001 93.979999) (end 97.790001 63.518051) (layer "Edge.Cuts") (width 0.1))
 (gr_arc (start 115.551949 93.979999) (mid 115.179975 94.878025) (end 114.281949 95.249999) (layer "Edge.Cuts") (width 0.1))
 (gr_arc (start 99.060001 95.249999) (mid 98.161975 94.878025) (end 97.790001 93.979999) (layer "Edge.Cuts") (width 0.1))
 (gr_arc (start 97.790001 63.518051) (mid 98.161975 62.620025) (end 99.060001 62.248051) (layer "Edge.Cuts") (width 0.1))
 (segment (start 107.696 65.278) (end 108.458 66.04) (width 0.3) (layer "F.Cu") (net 12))
 (segment (start 104.648 66.04) (end 105.41 65.278) (width 0.3) (layer "F.Cu") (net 12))
 (segment (start 105.41 65.278) (end 107.696 65.278) (width 0.3) (layer "F.Cu") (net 12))
 (segment (start 108.458 66.04) (end 108.458 67.056) (width 0.3) (layer "F.Cu") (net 12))
 (segment (start 104.29 69.183478) (end 104.29 68.33) (width 0.3) (layer "F.Cu") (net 12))
 (segment (start 104.29 68.33) (end 104.29 67.668) (width 0.3) (layer "F.Cu") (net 12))
 (segment (start 108.458 67.056) (end 108.458 67.698) (width 0.3) (layer "F.Cu") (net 12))
 (segment (start 103.148 70.5245) (end 103.148 70.325478) (width 0.3) (layer "F.Cu") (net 12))
 (segment (start 109.474 66.04) (end 114.3 66.04) (width 0.3) (layer "F.Cu") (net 12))
 (segment (start 104.648 67.31) (end 104.648 66.04) (width 0.3) (layer "F.Cu") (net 12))
 (segment (start 104.29 67.668) (end 104.648 67.31) (width 0.3) (layer "F.Cu") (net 12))
 (segment (start 103.148 70.325478) (end 104.29 69.183478) (width 0.3) (layer "F.Cu") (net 12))
 (segment (start 108.458 67.698) (end 109.09 68.33) (width 0.3) (layer "F.Cu") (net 12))
 (segment (start 108.458 67.056) (end 109.474 66.04) (width 0.3) (layer "F.Cu") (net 12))
 (segment (start 107.94 68.33) (end 107.94 67.3) (width 0.15) (layer "F.Cu") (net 15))
 (segment (start 107.94 67.3) (end 107.696 67.056) (width 0.15) (layer "F.Cu") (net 15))
 (via (at 107.696 67.056) (size 0.6) (drill 0.35) (layers "F.Cu" "B.Cu") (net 15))
 (segment (start 107.696 65.97) (end 107.596 65.87) (width 0.15) (layer "B.Cu") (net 15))
 (segment (start 107.696 67.056) (end 107.696 65.97) (width 0.15) (layer "B.Cu") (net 15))
 (segment (start 105.41 67.86) (end 105.41 67.056) (width 0.15) (layer "F.Cu") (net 16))
 (segment (start 104.94 68.33) (end 105.41 67.86) (width 0.15) (layer "F.Cu") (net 16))
 (via (at 105.41 67.056) (size 0.6) (drill 0.35) (layers "F.Cu" "B.Cu") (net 16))
 (segment (start 105.41 66.732) (end 104.548 65.87) (width 0.15) (layer "B.Cu") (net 16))
 (segment (start 105.41 67.056) (end 105.41 66.732) (width 0.15) (layer "B.Cu") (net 16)))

